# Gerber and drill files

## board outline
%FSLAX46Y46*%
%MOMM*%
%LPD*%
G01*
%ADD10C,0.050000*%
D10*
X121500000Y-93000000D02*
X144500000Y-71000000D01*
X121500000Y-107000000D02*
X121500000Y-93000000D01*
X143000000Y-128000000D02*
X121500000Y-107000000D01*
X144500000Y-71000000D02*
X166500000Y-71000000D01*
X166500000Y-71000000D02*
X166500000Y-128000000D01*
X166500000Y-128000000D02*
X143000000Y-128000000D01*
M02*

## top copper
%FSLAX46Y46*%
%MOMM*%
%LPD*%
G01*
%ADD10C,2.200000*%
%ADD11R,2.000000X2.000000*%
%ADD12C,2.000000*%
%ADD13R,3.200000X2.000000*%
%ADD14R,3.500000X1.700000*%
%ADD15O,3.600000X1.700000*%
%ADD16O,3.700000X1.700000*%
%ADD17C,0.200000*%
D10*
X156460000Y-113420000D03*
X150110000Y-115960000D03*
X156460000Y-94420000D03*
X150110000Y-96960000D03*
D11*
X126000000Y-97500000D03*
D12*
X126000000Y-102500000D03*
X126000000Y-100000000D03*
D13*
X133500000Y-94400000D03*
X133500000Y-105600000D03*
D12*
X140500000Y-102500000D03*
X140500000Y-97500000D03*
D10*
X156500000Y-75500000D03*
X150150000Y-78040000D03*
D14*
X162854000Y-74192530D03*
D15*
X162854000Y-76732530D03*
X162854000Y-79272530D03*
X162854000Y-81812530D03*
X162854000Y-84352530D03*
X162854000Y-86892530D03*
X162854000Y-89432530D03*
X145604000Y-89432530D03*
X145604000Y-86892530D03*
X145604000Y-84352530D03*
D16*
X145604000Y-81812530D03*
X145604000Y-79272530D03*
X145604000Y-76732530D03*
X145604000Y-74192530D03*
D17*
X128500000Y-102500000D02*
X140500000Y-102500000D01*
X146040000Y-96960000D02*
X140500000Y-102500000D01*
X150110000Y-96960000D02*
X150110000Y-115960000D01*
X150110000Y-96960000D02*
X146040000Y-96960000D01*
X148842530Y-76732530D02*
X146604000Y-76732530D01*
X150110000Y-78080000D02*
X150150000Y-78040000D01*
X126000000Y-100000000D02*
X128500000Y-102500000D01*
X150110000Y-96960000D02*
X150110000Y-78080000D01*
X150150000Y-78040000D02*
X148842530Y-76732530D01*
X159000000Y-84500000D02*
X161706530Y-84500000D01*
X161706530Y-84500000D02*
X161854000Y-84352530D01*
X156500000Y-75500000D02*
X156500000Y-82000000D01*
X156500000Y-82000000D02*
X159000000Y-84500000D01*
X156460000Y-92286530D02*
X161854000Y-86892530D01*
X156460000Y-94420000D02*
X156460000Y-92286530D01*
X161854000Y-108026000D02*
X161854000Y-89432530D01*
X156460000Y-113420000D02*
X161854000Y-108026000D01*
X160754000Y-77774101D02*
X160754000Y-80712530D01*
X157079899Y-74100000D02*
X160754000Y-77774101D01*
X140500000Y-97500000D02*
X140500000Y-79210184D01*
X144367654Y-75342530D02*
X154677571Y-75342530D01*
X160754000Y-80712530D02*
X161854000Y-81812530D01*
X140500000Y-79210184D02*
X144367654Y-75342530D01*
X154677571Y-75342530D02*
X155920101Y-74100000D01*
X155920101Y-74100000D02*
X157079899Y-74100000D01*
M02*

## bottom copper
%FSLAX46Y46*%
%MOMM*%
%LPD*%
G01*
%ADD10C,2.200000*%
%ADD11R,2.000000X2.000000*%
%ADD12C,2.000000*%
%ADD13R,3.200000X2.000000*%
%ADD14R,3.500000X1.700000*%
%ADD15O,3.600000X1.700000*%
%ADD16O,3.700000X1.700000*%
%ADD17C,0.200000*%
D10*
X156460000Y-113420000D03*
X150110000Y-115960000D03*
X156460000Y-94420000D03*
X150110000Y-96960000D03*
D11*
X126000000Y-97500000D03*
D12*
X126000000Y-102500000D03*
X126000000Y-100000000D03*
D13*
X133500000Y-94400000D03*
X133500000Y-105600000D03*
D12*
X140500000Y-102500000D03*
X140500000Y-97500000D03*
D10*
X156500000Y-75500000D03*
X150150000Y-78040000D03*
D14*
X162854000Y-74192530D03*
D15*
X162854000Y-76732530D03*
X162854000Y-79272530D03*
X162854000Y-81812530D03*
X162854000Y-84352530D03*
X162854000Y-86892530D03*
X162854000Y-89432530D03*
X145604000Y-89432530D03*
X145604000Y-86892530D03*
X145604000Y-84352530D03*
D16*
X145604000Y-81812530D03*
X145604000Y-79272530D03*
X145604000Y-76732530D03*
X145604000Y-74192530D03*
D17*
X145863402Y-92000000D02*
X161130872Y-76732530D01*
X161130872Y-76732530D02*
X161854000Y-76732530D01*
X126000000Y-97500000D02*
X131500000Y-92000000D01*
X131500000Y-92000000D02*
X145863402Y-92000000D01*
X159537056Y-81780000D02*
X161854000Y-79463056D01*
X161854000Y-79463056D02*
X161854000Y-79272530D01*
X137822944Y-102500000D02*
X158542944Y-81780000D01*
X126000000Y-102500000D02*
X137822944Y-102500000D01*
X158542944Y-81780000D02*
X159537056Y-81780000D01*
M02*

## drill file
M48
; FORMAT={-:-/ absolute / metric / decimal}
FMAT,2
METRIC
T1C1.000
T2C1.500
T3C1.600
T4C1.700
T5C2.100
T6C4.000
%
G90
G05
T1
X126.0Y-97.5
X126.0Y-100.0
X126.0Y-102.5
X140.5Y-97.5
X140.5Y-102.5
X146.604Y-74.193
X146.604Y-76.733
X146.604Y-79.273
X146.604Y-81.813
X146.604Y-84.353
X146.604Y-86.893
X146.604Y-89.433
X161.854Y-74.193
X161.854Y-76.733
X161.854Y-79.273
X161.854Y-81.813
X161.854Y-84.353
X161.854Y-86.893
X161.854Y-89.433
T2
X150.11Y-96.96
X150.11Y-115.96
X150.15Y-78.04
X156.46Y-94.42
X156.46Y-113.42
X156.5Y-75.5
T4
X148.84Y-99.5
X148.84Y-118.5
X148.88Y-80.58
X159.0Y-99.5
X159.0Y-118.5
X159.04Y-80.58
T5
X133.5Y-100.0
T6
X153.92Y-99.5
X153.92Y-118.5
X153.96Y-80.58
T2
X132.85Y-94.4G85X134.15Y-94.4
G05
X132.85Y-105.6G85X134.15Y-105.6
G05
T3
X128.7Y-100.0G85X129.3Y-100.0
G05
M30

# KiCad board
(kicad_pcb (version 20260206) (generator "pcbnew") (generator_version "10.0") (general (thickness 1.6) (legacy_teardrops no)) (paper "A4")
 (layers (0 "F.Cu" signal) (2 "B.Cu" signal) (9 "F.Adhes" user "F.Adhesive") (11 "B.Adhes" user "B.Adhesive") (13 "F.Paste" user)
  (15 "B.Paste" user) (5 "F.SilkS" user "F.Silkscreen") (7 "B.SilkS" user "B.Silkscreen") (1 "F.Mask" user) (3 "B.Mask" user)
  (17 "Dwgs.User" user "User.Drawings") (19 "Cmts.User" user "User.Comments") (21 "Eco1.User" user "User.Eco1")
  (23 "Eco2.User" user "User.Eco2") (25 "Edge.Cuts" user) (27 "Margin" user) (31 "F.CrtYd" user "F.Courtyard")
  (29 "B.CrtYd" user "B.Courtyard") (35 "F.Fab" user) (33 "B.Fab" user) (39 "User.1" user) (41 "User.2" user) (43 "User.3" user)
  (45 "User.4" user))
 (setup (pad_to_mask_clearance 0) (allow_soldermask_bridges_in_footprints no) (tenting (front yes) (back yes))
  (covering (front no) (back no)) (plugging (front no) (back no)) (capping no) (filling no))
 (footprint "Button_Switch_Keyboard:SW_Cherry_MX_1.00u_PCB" (layer "F.Cu") (at 156.46 113.42)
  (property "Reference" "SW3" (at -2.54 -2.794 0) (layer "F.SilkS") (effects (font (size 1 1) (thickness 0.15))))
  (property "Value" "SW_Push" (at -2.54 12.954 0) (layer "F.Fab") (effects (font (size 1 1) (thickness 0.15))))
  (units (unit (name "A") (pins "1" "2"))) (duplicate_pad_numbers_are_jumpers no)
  (pad "" np_thru_hole circle (at -7.62 5.08) (size 1.7 1.7) (drill 1.7) (layers "*.Cu" "*.Mask"))
  (pad "" np_thru_hole circle (at -2.54 5.08) (size 4 4) (drill 4) (layers "*.Cu" "*.Mask"))
  (pad "" np_thru_hole circle (at 2.54 5.08) (size 1.7 1.7) (drill 1.7) (layers "*.Cu" "*.Mask"))
  (pad "1" thru_hole circle (at 0 0) (size 2.2 2.2) (drill 1.5) (layers "*.Cu" "*.Mask") (remove_unused_layers no)
   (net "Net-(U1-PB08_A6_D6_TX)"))
  (pad "2" thru_hole circle (at -6.35 2.54) (size 2.2 2.2) (drill 1.5) (layers "*.Cu" "*.Mask") (remove_unused_layers no) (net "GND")))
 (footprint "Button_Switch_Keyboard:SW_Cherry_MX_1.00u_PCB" (layer "F.Cu") (at 156.46 94.42)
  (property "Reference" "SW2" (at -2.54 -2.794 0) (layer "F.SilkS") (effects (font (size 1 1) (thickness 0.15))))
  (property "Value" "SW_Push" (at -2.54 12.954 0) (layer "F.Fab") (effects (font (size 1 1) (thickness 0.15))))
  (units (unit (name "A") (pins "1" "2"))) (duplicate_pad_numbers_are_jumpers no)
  (pad "" np_thru_hole circle (at -7.62 5.08) (size 1.7 1.7) (drill 1.7) (layers "*.Cu" "*.Mask"))
  (pad "" np_thru_hole circle (at -2.54 5.08) (size 4 4) (drill 4) (layers "*.Cu" "*.Mask"))
  (pad "" np_thru_hole circle (at 2.54 5.08) (size 1.7 1.7) (drill 1.7) (layers "*.Cu" "*.Mask"))
  (pad "1" thru_hole circle (at 0 0) (size 2.2 2.2) (drill 1.5) (layers "*.Cu" "*.Mask") (remove_unused_layers no)
   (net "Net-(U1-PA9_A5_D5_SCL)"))
  (pad "2" thru_hole circle (at -6.35 2.54) (size 2.2 2.2) (drill 1.5) (layers "*.Cu" "*.Mask") (remove_unused_layers no) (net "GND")))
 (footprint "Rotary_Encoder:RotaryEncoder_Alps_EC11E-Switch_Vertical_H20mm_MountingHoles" (layer "F.Cu") (at 126 97.5)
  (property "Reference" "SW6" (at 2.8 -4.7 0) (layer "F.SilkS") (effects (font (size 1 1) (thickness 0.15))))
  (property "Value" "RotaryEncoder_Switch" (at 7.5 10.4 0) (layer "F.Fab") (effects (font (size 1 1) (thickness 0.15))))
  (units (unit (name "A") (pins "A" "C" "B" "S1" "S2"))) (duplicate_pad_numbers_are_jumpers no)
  (pad "" np_thru_hole oval (at 3 2.5) (size 2.2 1.6) (drill oval 2.2 1.6) (layers "*.Mask"))
  (pad "" np_thru_hole circle (at 7.5 2.5) (size 2.1 2.1) (drill 2.1) (layers "*.Mask"))
  (pad "A" thru_hole rect (at 0 0) (size 2 2) (drill 1) (layers "*.Cu" "*.Mask") (remove_unused_layers no) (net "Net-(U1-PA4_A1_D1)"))
  (pad "B" thru_hole circle (at 0 5) (size 2 2) (drill 1) (layers "*.Cu" "*.Mask") (remove_unused_layers no) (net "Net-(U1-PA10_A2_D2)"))
  (pad "C" thru_hole circle (at 0 2.5) (size 2 2) (drill 1) (layers "*.Cu" "*.Mask") (remove_unused_layers no) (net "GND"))
  (pad "MP" thru_hole rect (at 7.5 -3.1) (size 3.2 2) (drill oval 2.8 1.5) (layers "*.Cu" "*.Mask") (remove_unused_layers no))
  (pad "MP" thru_hole rect (at 7.5 8.1) (size 3.2 2) (drill oval 2.8 1.5) (layers "*.Cu" "*.Mask") (remove_unused_layers no))
  (pad "S1" thru_hole circle (at 14.5 5) (size 2 2) (drill 1) (layers "*.Cu" "*.Mask") (remove_unused_layers no) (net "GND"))
  (pad "S2" thru_hole circle (at 14.5 0) (size 2 2) (drill 1) (layers "*.Cu" "*.Mask") (remove_unused_layers no) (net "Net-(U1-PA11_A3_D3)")))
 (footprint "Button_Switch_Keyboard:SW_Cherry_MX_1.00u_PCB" (layer "F.Cu") (at 156.5 75.5)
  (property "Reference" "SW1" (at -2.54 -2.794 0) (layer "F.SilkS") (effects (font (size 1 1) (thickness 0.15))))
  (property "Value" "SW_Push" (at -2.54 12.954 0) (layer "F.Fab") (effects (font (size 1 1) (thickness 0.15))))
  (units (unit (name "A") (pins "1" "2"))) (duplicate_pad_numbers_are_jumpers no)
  (pad "" np_thru_hole circle (at -7.62 5.08) (size 1.7 1.7) (drill 1.7) (layers "*.Cu" "*.Mask"))
  (pad "" np_thru_hole circle (at -2.54 5.08) (size 4 4) (drill 4) (layers "*.Cu" "*.Mask"))
  (pad "" np_thru_hole circle (at 2.54 5.08) (size 1.7 1.7) (drill 1.7) (layers "*.Cu" "*.Mask"))
  (pad "1" thru_hole circle (at 0 0) (size 2.2 2.2) (drill 1.5) (layers "*.Cu" "*.Mask") (remove_unused_layers no)
   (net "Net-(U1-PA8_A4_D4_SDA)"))
  (pad "2" thru_hole circle (at -6.35 2.54) (size 2.2 2.2) (drill 1.5) (layers "*.Cu" "*.Mask") (remove_unused_layers no) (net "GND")))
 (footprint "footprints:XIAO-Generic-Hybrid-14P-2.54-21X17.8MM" (layer "B.Cu") (at 154.229 81.81253 180)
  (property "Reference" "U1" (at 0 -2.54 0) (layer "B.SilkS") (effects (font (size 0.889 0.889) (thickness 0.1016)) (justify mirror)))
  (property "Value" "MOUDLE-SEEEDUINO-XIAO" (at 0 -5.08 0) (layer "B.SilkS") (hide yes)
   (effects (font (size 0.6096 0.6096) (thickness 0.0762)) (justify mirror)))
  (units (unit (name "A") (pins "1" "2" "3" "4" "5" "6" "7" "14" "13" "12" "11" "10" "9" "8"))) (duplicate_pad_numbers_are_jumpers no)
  (pad "1" thru_hole rect (at -7.625 7.62 180) (size 3.5 1.7) (drill 1 (offset -1 0)) (layers "*.Cu" "*.Mask") (remove_unused_layers no)
   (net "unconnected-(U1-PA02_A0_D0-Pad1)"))
  (pad "2" thru_hole oval (at -7.625 5.08 180) (size 3.6 1.7) (drill 1 (offset -1 0)) (layers "*.Cu" "*.Mask") (remove_unused_layers no)
   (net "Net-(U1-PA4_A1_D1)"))
  (pad "3" thru_hole oval (at -7.625 2.54 180) (size 3.6 1.7) (drill 1 (offset -1 0)) (layers "*.Cu" "*.Mask") (remove_unused_layers no)
   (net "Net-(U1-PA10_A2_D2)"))
  (pad "4" thru_hole oval (at -7.625 0 180) (size 3.6 1.7) (drill 1 (offset -1 0)) (layers "*.Cu" "*.Mask") (remove_unused_layers no)
   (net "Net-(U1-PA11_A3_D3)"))
  (pad "5" thru_hole oval (at -7.625 -2.54 180) (size 3.6 1.7) (drill 1 (offset -1 0)) (layers "*.Cu" "*.Mask") (remove_unused_layers no)
   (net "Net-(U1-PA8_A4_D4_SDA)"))
  (pad "6" thru_hole oval (at -7.625 -5.08) (size 3.6 1.7) (drill 1 (offset 1 0)) (layers "*.Cu" "*.Mask") (remove_unused_layers no)
   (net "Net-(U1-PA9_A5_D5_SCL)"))
  (pad "7" thru_hole oval (at -7.625 -7.62 180) (size 3.6 1.7) (drill 1 (offset -1 0)) (layers "*.Cu" "*.Mask") (remove_unused_layers no)
   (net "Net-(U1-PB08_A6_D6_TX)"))
  (pad "8" thru_hole oval (at 7.625 -7.62 180) (size 3.6 1.7) (drill 1 (offset 1 0)) (layers "*.Cu" "*.Mask") (remove_unused_layers no)
   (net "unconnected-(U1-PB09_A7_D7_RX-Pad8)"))
  (pad "9" thru_hole oval (at 7.625 -5.08 180) (size 3.6 1.7) (drill 1 (offset 1 0)) (layers "*.Cu" "*.Mask") (remove_unused_layers no)
   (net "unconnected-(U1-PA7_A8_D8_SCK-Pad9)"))
  (pad "10" thru_hole oval (at 7.625 -2.54 180) (size 3.6 1.7) (drill 1 (offset 1 0)) (layers "*.Cu" "*.Mask") (remove_unused_layers no)
   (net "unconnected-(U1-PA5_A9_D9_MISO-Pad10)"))
  (pad "11" thru_hole oval (at 7.625 0 180) (size 3.7 1.7) (drill 1 (offset 1 0)) (layers "*.Cu" "*.Mask") (remove_unused_layers no)
   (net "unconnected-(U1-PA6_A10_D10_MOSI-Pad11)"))
  (pad "12" thru_hole oval (at 7.625 2.54 180) (size 3.7 1.7) (drill 1 (offset 1 0)) (layers "*.Cu" "*.Mask") (remove_unused_layers no)
   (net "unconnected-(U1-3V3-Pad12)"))
  (pad "13" thru_hole oval (at 7.625 5.08 180) (size 3.7 1.7) (drill 1 (offset 1 0)) (layers "*.Cu" "*.Mask") (remove_unused_layers no)
   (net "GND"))
  (pad "14" thru_hole oval (at 7.625 7.62 180) (size 3.7 1.7) (drill 1 (offset 1 0)) (layers "*.Cu" "*.Mask") (remove_unused_layers no)
   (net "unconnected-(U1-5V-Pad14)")))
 (gr_line (start 121.5 93) (end 144.5 71) (stroke (width 0.05) (type default)) (layer "Edge.Cuts"))
 (gr_line (start 121.5 107) (end 121.5 93) (stroke (width 0.05) (type default)) (layer "Edge.Cuts"))
 (gr_line (start 143 128) (end 121.5 107) (stroke (width 0.05) (type default)) (layer "Edge.Cuts"))
 (gr_line (start 144.5 71) (end 166.5 71) (stroke (width 0.05) (type default)) (layer "Edge.Cuts"))
 (gr_line (start 166.5 71) (end 166.5 128) (stroke (width 0.05) (type default)) (layer "Edge.Cuts"))
 (gr_line (start 166.5 128) (end 143 128) (stroke (width 0.05) (type default)) (layer "Edge.Cuts"))
 (segment (start 128.5 102.5) (end 140.5 102.5) (width 0.2) (layer "F.Cu") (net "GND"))
 (segment (start 146.04 96.96) (end 140.5 102.5) (width 0.2) (layer "F.Cu") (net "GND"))
 (segment (start 150.11 96.96) (end 150.11 115.96) (width 0.2) (layer "F.Cu") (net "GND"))
 (segment (start 150.11 96.96) (end 146.04 96.96) (width 0.2) (layer "F.Cu") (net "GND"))
 (segment (start 148.84253 76.73253) (end 146.604 76.73253) (width 0.2) (layer "F.Cu") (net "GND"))
 (segment (start 150.11 78.08) (end 150.15 78.04) (width 0.2) (layer "F.Cu") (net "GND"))
 (segment (start 126 100) (end 128.5 102.5) (width 0.2) (layer "F.Cu") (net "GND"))
 (segment (start 150.11 96.96) (end 150.11 78.08) (width 0.2) (layer "F.Cu") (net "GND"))
 (segment (start 150.15 78.04) (end 148.84253 76.73253) (width 0.2) (layer "F.Cu") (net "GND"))
 (segment (start 159 84.5) (end 161.70653 84.5) (width 0.2) (layer "F.Cu") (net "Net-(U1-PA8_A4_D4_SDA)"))
 (segment (start 161.70653 84.5) (end 161.854 84.35253) (width 0.2) (layer "F.Cu") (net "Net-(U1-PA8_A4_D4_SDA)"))
 (segment (start 156.5 75.5) (end 156.5 82) (width 0.2) (layer "F.Cu") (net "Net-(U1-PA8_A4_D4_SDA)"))
 (segment (start 156.5 82) (end 159 84.5) (width 0.2) (layer "F.Cu") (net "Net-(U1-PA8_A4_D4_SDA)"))
 (segment (start 156.46 92.28653) (end 161.854 86.89253) (width 0.2) (layer "F.Cu") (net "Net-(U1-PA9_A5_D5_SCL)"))
 (segment (start 156.46 94.42) (end 156.46 92.28653) (width 0.2) (layer "F.Cu") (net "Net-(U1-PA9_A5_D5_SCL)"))
 (segment (start 161.854 108.026) (end 161.854 89.43253) (width 0.2) (layer "F.Cu") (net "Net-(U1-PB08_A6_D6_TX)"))
 (segment (start 156.46 113.42) (end 161.854 108.026) (width 0.2) (layer "F.Cu") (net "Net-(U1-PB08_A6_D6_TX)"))
 (segment (start 145.863402 92) (end 161.130872 76.73253) (width 0.2) (layer "B.Cu") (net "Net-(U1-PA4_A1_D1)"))
 (segment (start 161.130872 76.73253) (end 161.854 76.73253) (width 0.2) (layer "B.Cu") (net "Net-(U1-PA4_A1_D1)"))
 (segment (start 126 97.5) (end 131.5 92) (width 0.2) (layer "B.Cu") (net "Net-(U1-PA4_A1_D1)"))
 (segment (start 131.5 92) (end 145.863402 92) (width 0.2) (layer "B.Cu") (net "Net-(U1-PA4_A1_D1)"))
 (segment (start 159.537056 81.78) (end 161.854 79.463056) (width 0.2) (layer "B.Cu") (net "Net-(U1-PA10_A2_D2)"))
 (segment (start 161.854 79.463056) (end 161.854 79.27253) (width 0.2) (layer "B.Cu") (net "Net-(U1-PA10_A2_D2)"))
 (segment (start 137.822944 102.5) (end 158.542944 81.78) (width 0.2) (layer "B.Cu") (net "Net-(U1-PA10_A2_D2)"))
 (segment (start 126 102.5) (end 137.822944 102.5) (width 0.2) (layer "B.Cu") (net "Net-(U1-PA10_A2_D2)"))
 (segment (start 158.542944 81.78) (end 159.537056 81.78) (width 0.2) (layer "B.Cu") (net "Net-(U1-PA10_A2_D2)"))
 (segment (start 160.754 77.774101) (end 160.754 80.71253) (width 0.2) (layer "F.Cu") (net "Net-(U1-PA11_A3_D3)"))
 (segment (start 157.079899 74.1) (end 160.754 77.774101) (width 0.2) (layer "F.Cu") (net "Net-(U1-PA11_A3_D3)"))
 (segment (start 140.5 97.5) (end 140.5 79.210184) (width 0.2) (layer "F.Cu") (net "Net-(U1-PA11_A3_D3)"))
 (segment (start 144.367654 75.34253) (end 154.677571 75.34253) (width 0.2) (layer "F.Cu") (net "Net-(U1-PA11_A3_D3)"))
 (segment (start 160.754 80.71253) (end 161.854 81.81253) (width 0.2) (layer "F.Cu") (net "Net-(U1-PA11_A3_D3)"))
 (segment (start 140.5 79.210184) (end 144.367654 75.34253) (width 0.2) (layer "F.Cu") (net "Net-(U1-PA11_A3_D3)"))
 (segment (start 154.677571 75.34253) (end 155.920101 74.1) (width 0.2) (layer "F.Cu") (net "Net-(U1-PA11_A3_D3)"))
 (segment (start 155.920101 74.1) (end 157.079899 74.1) (width 0.2) (layer "F.Cu") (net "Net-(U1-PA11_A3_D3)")))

